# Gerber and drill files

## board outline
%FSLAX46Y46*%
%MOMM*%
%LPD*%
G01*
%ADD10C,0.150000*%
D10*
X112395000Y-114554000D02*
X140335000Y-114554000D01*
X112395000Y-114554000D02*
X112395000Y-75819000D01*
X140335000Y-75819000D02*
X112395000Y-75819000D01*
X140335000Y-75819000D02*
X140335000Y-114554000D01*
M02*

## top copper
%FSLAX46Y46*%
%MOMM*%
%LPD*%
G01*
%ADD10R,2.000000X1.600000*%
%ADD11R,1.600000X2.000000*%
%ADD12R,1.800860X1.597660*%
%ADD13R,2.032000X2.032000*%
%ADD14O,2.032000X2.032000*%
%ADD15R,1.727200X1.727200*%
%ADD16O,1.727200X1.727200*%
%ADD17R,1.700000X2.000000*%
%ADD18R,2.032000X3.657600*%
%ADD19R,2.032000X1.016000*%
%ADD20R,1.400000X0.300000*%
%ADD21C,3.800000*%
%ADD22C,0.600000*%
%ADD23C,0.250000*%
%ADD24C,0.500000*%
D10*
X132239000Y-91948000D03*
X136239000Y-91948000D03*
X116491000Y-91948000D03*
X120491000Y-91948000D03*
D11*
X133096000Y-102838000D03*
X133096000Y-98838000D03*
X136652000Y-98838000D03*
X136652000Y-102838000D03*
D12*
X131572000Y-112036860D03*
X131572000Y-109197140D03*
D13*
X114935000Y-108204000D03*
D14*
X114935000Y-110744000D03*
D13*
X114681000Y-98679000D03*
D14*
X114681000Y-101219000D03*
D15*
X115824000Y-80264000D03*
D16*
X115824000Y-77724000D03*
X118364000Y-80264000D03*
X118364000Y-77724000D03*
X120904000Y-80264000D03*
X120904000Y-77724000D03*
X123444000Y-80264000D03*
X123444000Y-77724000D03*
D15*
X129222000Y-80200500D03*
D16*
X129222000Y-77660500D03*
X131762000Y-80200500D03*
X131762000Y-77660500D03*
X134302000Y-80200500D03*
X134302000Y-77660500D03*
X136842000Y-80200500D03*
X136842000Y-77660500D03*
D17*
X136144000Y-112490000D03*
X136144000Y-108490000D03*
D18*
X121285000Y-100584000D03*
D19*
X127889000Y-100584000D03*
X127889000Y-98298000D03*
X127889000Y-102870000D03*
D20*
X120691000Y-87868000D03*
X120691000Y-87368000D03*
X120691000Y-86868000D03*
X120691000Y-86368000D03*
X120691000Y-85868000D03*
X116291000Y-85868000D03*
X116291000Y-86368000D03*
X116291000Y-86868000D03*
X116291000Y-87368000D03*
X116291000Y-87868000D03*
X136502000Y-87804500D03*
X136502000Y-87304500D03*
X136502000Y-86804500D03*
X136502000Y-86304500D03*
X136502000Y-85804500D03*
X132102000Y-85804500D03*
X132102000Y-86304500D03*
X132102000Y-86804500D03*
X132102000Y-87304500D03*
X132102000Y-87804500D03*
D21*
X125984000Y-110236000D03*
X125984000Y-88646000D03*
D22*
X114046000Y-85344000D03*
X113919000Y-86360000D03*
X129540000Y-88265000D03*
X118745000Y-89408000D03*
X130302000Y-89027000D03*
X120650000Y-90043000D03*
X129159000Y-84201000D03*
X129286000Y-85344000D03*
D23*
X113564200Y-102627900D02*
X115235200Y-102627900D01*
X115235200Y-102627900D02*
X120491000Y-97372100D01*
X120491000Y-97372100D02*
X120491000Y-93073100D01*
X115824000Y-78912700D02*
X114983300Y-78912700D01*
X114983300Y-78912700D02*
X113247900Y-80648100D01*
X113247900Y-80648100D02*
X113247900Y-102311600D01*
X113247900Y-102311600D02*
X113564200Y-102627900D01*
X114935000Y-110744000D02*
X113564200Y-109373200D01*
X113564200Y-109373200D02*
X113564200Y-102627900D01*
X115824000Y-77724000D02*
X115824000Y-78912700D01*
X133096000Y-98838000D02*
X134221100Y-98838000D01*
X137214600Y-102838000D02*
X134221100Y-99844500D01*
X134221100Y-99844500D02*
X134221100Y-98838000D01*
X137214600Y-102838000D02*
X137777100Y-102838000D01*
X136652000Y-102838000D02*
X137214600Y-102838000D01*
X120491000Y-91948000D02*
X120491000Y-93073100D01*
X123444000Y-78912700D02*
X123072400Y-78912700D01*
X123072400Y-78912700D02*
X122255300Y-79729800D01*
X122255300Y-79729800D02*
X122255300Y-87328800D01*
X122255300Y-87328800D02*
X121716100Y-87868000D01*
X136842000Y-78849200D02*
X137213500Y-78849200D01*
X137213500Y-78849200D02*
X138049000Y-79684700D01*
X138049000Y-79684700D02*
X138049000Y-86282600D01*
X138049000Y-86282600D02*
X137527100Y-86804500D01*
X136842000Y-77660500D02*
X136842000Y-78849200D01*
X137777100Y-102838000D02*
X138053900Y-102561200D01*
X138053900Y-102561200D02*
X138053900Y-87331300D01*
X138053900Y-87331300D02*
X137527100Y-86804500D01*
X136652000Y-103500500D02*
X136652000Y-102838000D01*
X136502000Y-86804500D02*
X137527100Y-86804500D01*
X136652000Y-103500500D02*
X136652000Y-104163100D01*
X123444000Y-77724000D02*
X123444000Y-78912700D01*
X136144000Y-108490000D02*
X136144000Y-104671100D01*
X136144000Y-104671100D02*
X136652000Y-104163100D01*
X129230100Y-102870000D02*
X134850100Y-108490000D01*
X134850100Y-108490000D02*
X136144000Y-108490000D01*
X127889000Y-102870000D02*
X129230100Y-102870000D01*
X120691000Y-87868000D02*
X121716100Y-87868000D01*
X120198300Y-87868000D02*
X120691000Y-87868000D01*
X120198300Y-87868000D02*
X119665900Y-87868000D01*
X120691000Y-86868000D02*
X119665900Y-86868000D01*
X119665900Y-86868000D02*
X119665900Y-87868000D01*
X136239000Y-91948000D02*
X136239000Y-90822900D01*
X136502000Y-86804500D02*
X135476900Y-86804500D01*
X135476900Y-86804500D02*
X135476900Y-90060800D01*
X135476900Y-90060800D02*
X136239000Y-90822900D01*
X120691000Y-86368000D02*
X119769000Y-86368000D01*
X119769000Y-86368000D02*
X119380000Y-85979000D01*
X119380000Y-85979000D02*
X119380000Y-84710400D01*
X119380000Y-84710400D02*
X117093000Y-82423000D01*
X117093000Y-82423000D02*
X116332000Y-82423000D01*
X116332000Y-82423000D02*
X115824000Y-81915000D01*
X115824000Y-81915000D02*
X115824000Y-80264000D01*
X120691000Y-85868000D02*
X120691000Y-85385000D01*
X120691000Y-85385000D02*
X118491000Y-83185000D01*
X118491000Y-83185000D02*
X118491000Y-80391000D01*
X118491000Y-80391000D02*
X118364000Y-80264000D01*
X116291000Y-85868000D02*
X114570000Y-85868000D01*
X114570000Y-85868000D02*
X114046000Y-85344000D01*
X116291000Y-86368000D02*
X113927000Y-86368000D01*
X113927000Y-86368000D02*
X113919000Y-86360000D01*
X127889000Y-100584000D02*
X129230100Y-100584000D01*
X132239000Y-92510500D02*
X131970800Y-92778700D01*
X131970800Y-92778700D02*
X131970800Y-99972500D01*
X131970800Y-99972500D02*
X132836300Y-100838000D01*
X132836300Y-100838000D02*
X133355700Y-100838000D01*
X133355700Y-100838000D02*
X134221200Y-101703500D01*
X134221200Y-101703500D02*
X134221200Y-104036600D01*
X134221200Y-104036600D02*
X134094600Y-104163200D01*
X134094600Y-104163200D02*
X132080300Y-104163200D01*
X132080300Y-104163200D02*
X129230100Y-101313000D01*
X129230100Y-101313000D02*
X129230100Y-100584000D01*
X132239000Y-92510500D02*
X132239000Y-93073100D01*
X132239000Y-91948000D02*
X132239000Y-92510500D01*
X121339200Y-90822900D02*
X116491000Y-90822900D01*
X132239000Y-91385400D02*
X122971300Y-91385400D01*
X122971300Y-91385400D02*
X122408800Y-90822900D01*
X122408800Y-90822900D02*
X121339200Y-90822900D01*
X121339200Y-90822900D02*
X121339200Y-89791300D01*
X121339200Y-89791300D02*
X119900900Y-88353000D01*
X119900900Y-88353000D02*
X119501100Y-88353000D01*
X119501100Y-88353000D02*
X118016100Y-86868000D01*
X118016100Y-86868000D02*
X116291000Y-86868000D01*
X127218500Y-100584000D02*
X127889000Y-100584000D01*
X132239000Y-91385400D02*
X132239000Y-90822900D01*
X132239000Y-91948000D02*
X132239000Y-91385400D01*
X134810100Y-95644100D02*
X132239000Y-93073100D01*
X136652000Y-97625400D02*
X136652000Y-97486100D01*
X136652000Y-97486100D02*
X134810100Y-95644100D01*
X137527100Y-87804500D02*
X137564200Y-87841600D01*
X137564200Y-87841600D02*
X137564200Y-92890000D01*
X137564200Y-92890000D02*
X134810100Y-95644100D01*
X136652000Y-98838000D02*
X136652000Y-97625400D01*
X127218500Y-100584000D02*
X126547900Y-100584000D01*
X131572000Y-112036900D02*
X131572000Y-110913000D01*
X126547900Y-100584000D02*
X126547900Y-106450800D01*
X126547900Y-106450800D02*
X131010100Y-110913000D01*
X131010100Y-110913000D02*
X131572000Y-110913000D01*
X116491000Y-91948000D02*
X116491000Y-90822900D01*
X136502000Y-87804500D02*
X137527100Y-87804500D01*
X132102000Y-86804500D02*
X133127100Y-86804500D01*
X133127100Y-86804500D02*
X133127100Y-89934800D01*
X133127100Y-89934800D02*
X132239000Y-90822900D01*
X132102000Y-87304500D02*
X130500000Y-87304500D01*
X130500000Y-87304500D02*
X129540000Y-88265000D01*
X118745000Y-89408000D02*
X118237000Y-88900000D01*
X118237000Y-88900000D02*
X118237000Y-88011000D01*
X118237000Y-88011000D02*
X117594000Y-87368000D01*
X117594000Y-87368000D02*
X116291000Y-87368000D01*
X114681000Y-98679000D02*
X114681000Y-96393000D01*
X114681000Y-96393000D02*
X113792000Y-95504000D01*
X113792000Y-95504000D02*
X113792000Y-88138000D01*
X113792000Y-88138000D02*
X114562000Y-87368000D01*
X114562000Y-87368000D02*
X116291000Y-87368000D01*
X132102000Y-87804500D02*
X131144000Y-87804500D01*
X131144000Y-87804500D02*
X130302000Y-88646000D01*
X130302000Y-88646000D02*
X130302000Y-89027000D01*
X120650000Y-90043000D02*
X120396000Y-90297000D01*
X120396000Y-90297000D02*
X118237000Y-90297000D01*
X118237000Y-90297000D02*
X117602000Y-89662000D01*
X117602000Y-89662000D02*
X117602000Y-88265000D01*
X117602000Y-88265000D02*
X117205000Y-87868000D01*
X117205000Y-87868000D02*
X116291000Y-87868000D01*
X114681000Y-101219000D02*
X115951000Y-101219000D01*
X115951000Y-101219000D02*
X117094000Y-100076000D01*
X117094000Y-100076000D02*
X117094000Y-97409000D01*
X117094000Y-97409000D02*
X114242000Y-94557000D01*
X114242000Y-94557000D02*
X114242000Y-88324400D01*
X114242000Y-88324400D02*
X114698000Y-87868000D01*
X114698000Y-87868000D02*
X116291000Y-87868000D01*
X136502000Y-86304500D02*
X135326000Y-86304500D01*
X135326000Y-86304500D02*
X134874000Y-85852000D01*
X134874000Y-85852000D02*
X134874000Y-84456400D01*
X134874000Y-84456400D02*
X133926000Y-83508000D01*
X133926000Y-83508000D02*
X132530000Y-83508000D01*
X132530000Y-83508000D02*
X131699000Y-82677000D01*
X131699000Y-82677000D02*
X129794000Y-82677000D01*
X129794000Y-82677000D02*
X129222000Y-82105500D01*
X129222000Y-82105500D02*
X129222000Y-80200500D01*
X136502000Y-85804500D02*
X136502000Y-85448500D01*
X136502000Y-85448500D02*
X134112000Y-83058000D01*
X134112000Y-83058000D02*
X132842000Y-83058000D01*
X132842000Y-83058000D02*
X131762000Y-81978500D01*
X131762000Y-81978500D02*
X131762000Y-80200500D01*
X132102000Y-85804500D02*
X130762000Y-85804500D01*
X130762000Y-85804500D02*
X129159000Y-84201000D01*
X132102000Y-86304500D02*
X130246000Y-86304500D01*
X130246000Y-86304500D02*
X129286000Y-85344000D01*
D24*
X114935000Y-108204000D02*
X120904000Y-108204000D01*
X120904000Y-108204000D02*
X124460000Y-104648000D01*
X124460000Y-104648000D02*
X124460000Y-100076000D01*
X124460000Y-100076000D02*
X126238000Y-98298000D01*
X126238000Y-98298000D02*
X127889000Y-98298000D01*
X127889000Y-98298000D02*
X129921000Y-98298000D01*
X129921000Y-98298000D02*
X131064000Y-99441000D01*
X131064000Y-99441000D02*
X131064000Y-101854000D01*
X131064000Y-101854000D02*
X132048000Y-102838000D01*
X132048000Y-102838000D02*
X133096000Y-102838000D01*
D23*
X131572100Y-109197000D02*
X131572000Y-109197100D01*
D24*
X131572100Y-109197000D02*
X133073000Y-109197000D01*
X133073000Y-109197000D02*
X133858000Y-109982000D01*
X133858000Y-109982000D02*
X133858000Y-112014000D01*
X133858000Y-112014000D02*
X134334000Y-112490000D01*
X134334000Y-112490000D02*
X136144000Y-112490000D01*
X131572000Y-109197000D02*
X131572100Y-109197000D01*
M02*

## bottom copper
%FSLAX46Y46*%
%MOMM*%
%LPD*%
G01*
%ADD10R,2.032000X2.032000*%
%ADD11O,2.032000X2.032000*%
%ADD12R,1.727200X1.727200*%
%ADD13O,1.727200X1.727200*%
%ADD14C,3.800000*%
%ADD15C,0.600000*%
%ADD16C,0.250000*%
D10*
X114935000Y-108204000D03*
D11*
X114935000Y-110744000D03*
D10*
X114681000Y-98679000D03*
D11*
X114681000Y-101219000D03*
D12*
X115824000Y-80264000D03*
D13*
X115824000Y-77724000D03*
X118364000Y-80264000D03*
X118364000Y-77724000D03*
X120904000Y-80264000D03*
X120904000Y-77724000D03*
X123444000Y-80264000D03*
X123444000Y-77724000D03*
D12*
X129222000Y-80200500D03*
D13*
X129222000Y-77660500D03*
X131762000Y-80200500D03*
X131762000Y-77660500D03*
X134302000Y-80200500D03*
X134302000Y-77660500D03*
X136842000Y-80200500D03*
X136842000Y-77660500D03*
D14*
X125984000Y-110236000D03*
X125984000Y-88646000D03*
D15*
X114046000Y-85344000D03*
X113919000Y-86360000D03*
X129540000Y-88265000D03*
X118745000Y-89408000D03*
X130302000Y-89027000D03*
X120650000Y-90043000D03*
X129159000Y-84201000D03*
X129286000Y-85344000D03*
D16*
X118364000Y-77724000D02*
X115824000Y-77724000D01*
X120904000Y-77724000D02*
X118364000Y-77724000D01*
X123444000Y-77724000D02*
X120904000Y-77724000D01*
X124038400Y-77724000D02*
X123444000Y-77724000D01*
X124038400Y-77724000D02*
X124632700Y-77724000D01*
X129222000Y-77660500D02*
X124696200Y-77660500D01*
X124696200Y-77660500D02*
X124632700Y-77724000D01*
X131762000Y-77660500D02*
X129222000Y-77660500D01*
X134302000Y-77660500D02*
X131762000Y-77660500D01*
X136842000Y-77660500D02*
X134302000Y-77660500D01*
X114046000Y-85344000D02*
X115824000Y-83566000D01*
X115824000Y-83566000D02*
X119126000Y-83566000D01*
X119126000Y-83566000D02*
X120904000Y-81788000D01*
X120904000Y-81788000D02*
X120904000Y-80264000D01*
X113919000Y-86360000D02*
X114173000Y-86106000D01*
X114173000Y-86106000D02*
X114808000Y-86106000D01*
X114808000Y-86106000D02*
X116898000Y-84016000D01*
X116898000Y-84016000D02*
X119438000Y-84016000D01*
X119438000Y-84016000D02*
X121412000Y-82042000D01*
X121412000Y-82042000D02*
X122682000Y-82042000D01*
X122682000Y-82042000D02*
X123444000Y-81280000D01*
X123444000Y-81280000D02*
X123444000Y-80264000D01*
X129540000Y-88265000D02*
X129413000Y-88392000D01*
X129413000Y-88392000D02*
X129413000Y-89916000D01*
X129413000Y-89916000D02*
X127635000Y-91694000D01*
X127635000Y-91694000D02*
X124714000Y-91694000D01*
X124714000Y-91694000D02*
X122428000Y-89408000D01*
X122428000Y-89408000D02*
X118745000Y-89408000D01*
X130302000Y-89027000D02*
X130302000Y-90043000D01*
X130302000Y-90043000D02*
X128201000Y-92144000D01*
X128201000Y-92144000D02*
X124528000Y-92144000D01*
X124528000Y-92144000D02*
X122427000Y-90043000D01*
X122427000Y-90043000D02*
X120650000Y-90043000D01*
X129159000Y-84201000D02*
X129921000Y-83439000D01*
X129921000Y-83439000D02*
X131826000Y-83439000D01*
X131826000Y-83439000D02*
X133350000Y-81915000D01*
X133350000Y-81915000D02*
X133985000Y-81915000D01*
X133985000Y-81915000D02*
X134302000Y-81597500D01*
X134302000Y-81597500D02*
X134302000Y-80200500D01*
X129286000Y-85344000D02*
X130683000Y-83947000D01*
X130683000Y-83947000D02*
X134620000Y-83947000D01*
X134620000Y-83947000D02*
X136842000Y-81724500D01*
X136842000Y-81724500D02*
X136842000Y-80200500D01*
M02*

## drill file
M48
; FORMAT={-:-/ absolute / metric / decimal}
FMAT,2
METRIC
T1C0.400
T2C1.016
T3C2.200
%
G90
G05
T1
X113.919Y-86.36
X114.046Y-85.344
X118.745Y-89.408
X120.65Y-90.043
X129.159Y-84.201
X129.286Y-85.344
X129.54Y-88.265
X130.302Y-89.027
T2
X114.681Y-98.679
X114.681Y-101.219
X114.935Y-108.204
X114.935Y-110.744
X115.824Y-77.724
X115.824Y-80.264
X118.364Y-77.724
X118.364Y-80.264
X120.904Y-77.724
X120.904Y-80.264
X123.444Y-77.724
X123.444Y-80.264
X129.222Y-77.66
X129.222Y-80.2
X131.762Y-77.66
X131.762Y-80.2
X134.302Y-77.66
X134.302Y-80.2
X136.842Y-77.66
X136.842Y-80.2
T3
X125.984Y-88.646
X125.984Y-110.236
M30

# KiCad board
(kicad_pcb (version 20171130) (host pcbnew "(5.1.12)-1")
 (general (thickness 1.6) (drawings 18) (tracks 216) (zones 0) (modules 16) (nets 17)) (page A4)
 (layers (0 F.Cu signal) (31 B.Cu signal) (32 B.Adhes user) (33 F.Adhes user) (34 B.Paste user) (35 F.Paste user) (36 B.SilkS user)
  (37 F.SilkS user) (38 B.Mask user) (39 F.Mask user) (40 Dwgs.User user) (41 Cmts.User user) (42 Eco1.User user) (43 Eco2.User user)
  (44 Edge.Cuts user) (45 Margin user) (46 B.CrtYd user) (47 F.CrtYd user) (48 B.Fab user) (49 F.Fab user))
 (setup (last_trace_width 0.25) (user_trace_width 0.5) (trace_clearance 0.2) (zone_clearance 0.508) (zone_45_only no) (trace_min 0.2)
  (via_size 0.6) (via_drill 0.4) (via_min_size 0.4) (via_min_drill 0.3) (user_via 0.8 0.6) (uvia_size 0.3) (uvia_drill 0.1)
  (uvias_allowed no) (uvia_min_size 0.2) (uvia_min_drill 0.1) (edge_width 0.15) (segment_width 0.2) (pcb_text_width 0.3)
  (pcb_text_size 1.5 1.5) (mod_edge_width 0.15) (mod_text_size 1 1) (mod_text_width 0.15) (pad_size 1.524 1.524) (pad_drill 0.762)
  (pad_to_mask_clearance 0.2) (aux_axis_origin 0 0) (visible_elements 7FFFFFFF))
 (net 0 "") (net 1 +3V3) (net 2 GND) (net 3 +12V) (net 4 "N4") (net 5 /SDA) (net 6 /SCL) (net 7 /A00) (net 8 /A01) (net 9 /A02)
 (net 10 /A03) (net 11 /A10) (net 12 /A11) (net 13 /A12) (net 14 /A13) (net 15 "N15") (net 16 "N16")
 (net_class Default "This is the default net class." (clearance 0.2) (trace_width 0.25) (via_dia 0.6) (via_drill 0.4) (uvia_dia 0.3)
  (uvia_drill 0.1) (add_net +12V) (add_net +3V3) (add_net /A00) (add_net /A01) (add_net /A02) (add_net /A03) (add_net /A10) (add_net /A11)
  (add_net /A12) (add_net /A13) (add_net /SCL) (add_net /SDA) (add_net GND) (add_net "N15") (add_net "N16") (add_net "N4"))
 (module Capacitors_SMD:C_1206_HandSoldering (layer F.Cu) (at 134.239 91.948)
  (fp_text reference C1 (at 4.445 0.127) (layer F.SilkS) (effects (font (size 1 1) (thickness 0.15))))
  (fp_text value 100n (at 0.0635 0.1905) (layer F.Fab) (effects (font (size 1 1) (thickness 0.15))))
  (pad 1 smd rect (at -2 0) (size 2 1.6) (layers F.Cu F.Paste F.Mask) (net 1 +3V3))
  (pad 2 smd rect (at 2 0) (size 2 1.6) (layers F.Cu F.Paste F.Mask) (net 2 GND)))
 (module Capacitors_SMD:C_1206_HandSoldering (layer F.Cu) (at 118.491 91.948)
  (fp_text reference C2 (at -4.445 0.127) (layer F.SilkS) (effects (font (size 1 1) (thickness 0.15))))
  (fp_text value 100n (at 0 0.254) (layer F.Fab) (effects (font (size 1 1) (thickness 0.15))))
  (pad 1 smd rect (at -2 0) (size 2 1.6) (layers F.Cu F.Paste F.Mask) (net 1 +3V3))
  (pad 2 smd rect (at 2 0) (size 2 1.6) (layers F.Cu F.Paste F.Mask) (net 2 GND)))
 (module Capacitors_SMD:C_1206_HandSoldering (layer F.Cu) (at 133.096 100.838 90)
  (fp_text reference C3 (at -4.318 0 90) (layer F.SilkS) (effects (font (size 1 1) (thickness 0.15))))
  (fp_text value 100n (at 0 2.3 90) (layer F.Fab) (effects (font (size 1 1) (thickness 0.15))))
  (pad 1 smd rect (at -2 0 90) (size 2 1.6) (layers F.Cu F.Paste F.Mask) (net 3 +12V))
  (pad 2 smd rect (at 2 0 90) (size 2 1.6) (layers F.Cu F.Paste F.Mask) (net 2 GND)))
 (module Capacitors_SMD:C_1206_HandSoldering (layer F.Cu) (at 136.652 100.838 270)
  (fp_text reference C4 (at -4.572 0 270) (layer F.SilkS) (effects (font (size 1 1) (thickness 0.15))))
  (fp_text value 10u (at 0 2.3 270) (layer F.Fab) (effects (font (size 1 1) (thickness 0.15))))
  (pad 1 smd rect (at -2 0 270) (size 2 1.6) (layers F.Cu F.Paste F.Mask) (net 1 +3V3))
  (pad 2 smd rect (at 2 0 270) (size 2 1.6) (layers F.Cu F.Paste F.Mask) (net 2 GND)))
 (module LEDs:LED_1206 (layer F.Cu) (at 131.572 110.617 270)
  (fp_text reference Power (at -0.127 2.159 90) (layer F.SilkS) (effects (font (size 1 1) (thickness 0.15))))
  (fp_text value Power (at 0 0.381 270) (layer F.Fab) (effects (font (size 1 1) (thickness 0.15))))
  (pad 2 smd rect (at 1.41986 0 90) (size 1.59766 1.80086) (layers F.Cu F.Paste F.Mask) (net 1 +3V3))
  (pad 1 smd rect (at -1.41986 0 90) (size 1.59766 1.80086) (layers F.Cu F.Paste F.Mask) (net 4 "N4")))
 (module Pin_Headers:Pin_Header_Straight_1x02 (layer F.Cu) (at 114.935 108.204)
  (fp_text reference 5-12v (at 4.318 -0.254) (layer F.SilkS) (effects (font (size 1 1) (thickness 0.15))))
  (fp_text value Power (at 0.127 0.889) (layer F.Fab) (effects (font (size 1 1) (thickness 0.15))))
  (pad 1 thru_hole rect (at 0 0) (size 2.032 2.032) (drill 1.016) (layers *.Cu *.Mask F.SilkS) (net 3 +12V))
  (pad 2 thru_hole oval (at 0 2.54) (size 2.032 2.032) (drill 1.016) (layers *.Cu *.Mask F.SilkS) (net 2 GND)))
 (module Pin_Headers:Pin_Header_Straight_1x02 (layer F.Cu) (at 114.681 98.679)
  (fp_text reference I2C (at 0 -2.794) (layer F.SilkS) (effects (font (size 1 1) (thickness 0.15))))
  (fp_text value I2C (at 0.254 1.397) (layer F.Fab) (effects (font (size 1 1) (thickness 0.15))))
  (pad 1 thru_hole rect (at 0 0) (size 2.032 2.032) (drill 1.016) (layers *.Cu *.Mask F.SilkS) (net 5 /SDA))
  (pad 2 thru_hole oval (at 0 2.54) (size 2.032 2.032) (drill 1.016) (layers *.Cu *.Mask F.SilkS) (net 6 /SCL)))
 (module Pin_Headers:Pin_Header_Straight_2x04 (layer F.Cu) (at 115.824 80.264 90)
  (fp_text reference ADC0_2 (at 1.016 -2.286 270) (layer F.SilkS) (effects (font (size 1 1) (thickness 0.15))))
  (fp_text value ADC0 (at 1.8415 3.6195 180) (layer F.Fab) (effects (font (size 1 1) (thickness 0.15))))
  (pad 1 thru_hole rect (at 0 0 90) (size 1.7272 1.7272) (drill 1.016) (layers *.Cu *.Mask F.SilkS) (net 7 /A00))
  (pad 2 thru_hole oval (at 2.54 0 90) (size 1.7272 1.7272) (drill 1.016) (layers *.Cu *.Mask F.SilkS) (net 2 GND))
  (pad 3 thru_hole oval (at 0 2.54 90) (size 1.7272 1.7272) (drill 1.016) (layers *.Cu *.Mask F.SilkS) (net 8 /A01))
  (pad 4 thru_hole oval (at 2.54 2.54 90) (size 1.7272 1.7272) (drill 1.016) (layers *.Cu *.Mask F.SilkS) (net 2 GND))
  (pad 5 thru_hole oval (at 0 5.08 90) (size 1.7272 1.7272) (drill 1.016) (layers *.Cu *.Mask F.SilkS) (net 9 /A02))
  (pad 6 thru_hole oval (at 2.54 5.08 90) (size 1.7272 1.7272) (drill 1.016) (layers *.Cu *.Mask F.SilkS) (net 2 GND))
  (pad 7 thru_hole oval (at 0 7.62 90) (size 1.7272 1.7272) (drill 1.016) (layers *.Cu *.Mask F.SilkS) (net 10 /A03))
  (pad 8 thru_hole oval (at 2.54 7.62 90) (size 1.7272 1.7272) (drill 1.016) (layers *.Cu *.Mask F.SilkS) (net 2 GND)))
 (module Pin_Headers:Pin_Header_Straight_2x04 (layer F.Cu) (at 129.222 80.2005 90)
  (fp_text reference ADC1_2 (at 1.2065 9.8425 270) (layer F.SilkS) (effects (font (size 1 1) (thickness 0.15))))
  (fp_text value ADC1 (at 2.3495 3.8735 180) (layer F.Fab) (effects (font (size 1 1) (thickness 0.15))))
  (pad 1 thru_hole rect (at 0 0 90) (size 1.7272 1.7272) (drill 1.016) (layers *.Cu *.Mask F.SilkS) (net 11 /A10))
  (pad 2 thru_hole oval (at 2.54 0 90) (size 1.7272 1.7272) (drill 1.016) (layers *.Cu *.Mask F.SilkS) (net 2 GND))
  (pad 3 thru_hole oval (at 0 2.54 90) (size 1.7272 1.7272) (drill 1.016) (layers *.Cu *.Mask F.SilkS) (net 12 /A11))
  (pad 4 thru_hole oval (at 2.54 2.54 90) (size 1.7272 1.7272) (drill 1.016) (layers *.Cu *.Mask F.SilkS) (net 2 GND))
  (pad 5 thru_hole oval (at 0 5.08 90) (size 1.7272 1.7272) (drill 1.016) (layers *.Cu *.Mask F.SilkS) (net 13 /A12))
  (pad 6 thru_hole oval (at 2.54 5.08 90) (size 1.7272 1.7272) (drill 1.016) (layers *.Cu *.Mask F.SilkS) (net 2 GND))
  (pad 7 thru_hole oval (at 0 7.62 90) (size 1.7272 1.7272) (drill 1.016) (layers *.Cu *.Mask F.SilkS) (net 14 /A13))
  (pad 8 thru_hole oval (at 2.54 7.62 90) (size 1.7272 1.7272) (drill 1.016) (layers *.Cu *.Mask F.SilkS) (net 2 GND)))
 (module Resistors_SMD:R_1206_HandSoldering (layer F.Cu) (at 136.144 110.49 90)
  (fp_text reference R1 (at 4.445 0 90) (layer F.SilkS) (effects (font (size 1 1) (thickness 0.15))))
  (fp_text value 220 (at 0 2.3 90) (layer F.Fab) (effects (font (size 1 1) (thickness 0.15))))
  (pad 1 smd rect (at -2 0 90) (size 2 1.7) (layers F.Cu F.Paste F.Mask) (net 4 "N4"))
  (pad 2 smd rect (at 2 0 90) (size 2 1.7) (layers F.Cu F.Paste F.Mask) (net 2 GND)))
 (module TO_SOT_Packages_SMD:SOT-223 (layer F.Cu) (at 124.587 100.584 90)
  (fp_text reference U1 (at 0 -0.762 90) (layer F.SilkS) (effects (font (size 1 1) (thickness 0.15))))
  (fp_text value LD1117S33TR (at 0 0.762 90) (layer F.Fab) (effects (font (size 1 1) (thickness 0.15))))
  (pad 4 smd rect (at 0 -3.302 90) (size 3.6576 2.032) (layers F.Cu F.Paste F.Mask))
  (pad 2 smd rect (at 0 3.302 90) (size 1.016 2.032) (layers F.Cu F.Paste F.Mask) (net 1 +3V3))
  (pad 3 smd rect (at 2.286 3.302 90) (size 1.016 2.032) (layers F.Cu F.Paste F.Mask) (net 3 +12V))
  (pad 1 smd rect (at -2.286 3.302 90) (size 1.016 2.032) (layers F.Cu F.Paste F.Mask) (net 2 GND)))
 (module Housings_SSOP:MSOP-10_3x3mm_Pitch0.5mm (layer F.Cu) (at 118.491 86.868 180)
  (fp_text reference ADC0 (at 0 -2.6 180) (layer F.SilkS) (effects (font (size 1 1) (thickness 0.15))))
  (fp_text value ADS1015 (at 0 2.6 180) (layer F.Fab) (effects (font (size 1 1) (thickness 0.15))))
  (pad 1 smd rect (at -2.2 -1 180) (size 1.4 0.3) (layers F.Cu F.Paste F.Mask) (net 2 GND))
  (pad 2 smd rect (at -2.2 -0.5 180) (size 1.4 0.3) (layers F.Cu F.Paste F.Mask) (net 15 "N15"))
  (pad 3 smd rect (at -2.2 0 180) (size 1.4 0.3) (layers F.Cu F.Paste F.Mask) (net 2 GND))
  (pad 4 smd rect (at -2.2 0.5 180) (size 1.4 0.3) (layers F.Cu F.Paste F.Mask) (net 7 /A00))
  (pad 5 smd rect (at -2.2 1 180) (size 1.4 0.3) (layers F.Cu F.Paste F.Mask) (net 8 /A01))
  (pad 6 smd rect (at 2.2 1 180) (size 1.4 0.3) (layers F.Cu F.Paste F.Mask) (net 9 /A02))
  (pad 7 smd rect (at 2.2 0.5 180) (size 1.4 0.3) (layers F.Cu F.Paste F.Mask) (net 10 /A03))
  (pad 8 smd rect (at 2.2 0 180) (size 1.4 0.3) (layers F.Cu F.Paste F.Mask) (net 1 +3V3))
  (pad 9 smd rect (at 2.2 -0.5 180) (size 1.4 0.3) (layers F.Cu F.Paste F.Mask) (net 5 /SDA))
  (pad 10 smd rect (at 2.2 -1 180) (size 1.4 0.3) (layers F.Cu F.Paste F.Mask) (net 6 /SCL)))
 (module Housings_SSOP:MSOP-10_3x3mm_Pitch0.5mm (layer F.Cu) (at 134.302 86.8045 180)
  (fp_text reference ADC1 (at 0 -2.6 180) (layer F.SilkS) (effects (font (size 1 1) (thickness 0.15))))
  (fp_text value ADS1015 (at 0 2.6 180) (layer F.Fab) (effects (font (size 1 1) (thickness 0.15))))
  (pad 1 smd rect (at -2.2 -1 180) (size 1.4 0.3) (layers F.Cu F.Paste F.Mask) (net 1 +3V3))
  (pad 2 smd rect (at -2.2 -0.5 180) (size 1.4 0.3) (layers F.Cu F.Paste F.Mask) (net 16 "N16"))
  (pad 3 smd rect (at -2.2 0 180) (size 1.4 0.3) (layers F.Cu F.Paste F.Mask) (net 2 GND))
  (pad 4 smd rect (at -2.2 0.5 180) (size 1.4 0.3) (layers F.Cu F.Paste F.Mask) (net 11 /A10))
  (pad 5 smd rect (at -2.2 1 180) (size 1.4 0.3) (layers F.Cu F.Paste F.Mask) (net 12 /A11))
  (pad 6 smd rect (at 2.2 1 180) (size 1.4 0.3) (layers F.Cu F.Paste F.Mask) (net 13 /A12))
  (pad 7 smd rect (at 2.2 0.5 180) (size 1.4 0.3) (layers F.Cu F.Paste F.Mask) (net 14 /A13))
  (pad 8 smd rect (at 2.2 0 180) (size 1.4 0.3) (layers F.Cu F.Paste F.Mask) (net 1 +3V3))
  (pad 9 smd rect (at 2.2 -0.5 180) (size 1.4 0.3) (layers F.Cu F.Paste F.Mask) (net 5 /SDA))
  (pad 10 smd rect (at 2.2 -1 180) (size 1.4 0.3) (layers F.Cu F.Paste F.Mask) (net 6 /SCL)))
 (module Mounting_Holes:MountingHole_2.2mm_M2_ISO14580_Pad (layer F.Cu) (at 125.984 110.236)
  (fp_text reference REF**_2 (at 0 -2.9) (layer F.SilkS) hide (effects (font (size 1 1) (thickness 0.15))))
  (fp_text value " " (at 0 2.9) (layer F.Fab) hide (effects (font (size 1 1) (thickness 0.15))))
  (pad 1 thru_hole circle (at 0 0) (size 3.8 3.8) (drill 2.2) (layers *.Cu *.Mask F.SilkS)))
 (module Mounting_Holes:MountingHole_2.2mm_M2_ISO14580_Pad (layer F.Cu) (at 125.984 88.646)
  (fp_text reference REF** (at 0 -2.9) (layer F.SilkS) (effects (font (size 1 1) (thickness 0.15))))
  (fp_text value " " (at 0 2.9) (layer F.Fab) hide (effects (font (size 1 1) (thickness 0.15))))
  (pad 1 thru_hole circle (at 0 0) (size 3.8 3.8) (drill 2.2) (layers *.Cu *.Mask F.SilkS)))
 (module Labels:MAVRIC (layer B.Cu) (at 127.889 100.076 90)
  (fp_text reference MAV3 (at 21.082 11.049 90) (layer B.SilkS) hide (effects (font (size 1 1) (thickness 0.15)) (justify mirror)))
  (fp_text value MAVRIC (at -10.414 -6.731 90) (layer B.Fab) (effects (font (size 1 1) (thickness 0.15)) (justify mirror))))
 (gr_line (start 112.395 114.554) (end 140.335 114.554) (angle 90) (layer Edge.Cuts) (width 0.15))
 (gr_line (start 112.395 114.554) (end 112.395 75.819) (angle 90) (layer Edge.Cuts) (width 0.15))
 (gr_line (start 140.335 75.819) (end 112.395 75.819) (angle 90) (layer Edge.Cuts) (width 0.15))
 (gr_line (start 140.335 75.819) (end 140.335 114.554) (angle 90) (layer Edge.Cuts) (width 0.15))
 (segment (start 113.5642 102.6279) (end 115.2352 102.6279) (width 0.25) (layer F.Cu) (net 2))
 (segment (start 115.2352 102.6279) (end 120.491 97.3721) (width 0.25) (layer F.Cu) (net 2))
 (segment (start 120.491 97.3721) (end 120.491 93.0731) (width 0.25) (layer F.Cu) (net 2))
 (segment (start 115.824 78.9127) (end 114.9833 78.9127) (width 0.25) (layer F.Cu) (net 2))
 (segment (start 114.9833 78.9127) (end 113.2479 80.6481) (width 0.25) (layer F.Cu) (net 2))
 (segment (start 113.2479 80.6481) (end 113.2479 102.3116) (width 0.25) (layer F.Cu) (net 2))
 (segment (start 113.2479 102.3116) (end 113.5642 102.6279) (width 0.25) (layer F.Cu) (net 2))
 (segment (start 114.935 110.744) (end 113.5642 109.3732) (width 0.25) (layer F.Cu) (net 2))
 (segment (start 113.5642 109.3732) (end 113.5642 102.6279) (width 0.25) (layer F.Cu) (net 2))
 (segment (start 115.824 77.724) (end 115.824 78.9127) (width 0.25) (layer F.Cu) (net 2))
 (segment (start 133.096 98.838) (end 134.2211 98.838) (width 0.25) (layer F.Cu) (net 2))
 (segment (start 137.2146 102.838) (end 134.2211 99.8445) (width 0.25) (layer F.Cu) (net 2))
 (segment (start 134.2211 99.8445) (end 134.2211 98.838) (width 0.25) (layer F.Cu) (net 2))
 (segment (start 137.2146 102.838) (end 137.7771 102.838) (width 0.25) (layer F.Cu) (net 2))
 (segment (start 136.652 102.838) (end 137.2146 102.838) (width 0.25) (layer F.Cu) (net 2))
 (segment (start 120.491 91.948) (end 120.491 93.0731) (width 0.25) (layer F.Cu) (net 2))
 (segment (start 123.444 78.9127) (end 123.0724 78.9127) (width 0.25) (layer F.Cu) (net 2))
 (segment (start 123.0724 78.9127) (end 122.2553 79.7298) (width 0.25) (layer F.Cu) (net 2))
 (segment (start 122.2553 79.7298) (end 122.2553 87.3288) (width 0.25) (layer F.Cu) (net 2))
 (segment (start 122.2553 87.3288) (end 121.7161 87.868) (width 0.25) (layer F.Cu) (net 2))
 (segment (start 136.842 78.8492) (end 137.2135 78.8492) (width 0.25) (layer F.Cu) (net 2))
 (segment (start 137.2135 78.8492) (end 138.049 79.6847) (width 0.25) (layer F.Cu) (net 2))
 (segment (start 138.049 79.6847) (end 138.049 86.2826) (width 0.25) (layer F.Cu) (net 2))
 (segment (start 138.049 86.2826) (end 137.5271 86.8045) (width 0.25) (layer F.Cu) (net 2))
 (segment (start 136.842 77.6605) (end 136.842 78.8492) (width 0.25) (layer F.Cu) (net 2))
 (segment (start 137.7771 102.838) (end 138.0539 102.5612) (width 0.25) (layer F.Cu) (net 2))
 (segment (start 138.0539 102.5612) (end 138.0539 87.3313) (width 0.25) (layer F.Cu) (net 2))
 (segment (start 138.0539 87.3313) (end 137.5271 86.8045) (width 0.25) (layer F.Cu) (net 2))
 (segment (start 136.652 103.5005) (end 136.652 102.838) (width 0.25) (layer F.Cu) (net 2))
 (segment (start 136.502 86.8045) (end 137.5271 86.8045) (width 0.25) (layer F.Cu) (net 2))
 (segment (start 136.652 103.5005) (end 136.652 104.1631) (width 0.25) (layer F.Cu) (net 2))
 (segment (start 123.444 77.724) (end 123.444 78.9127) (width 0.25) (layer F.Cu) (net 2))
 (segment (start 118.364 77.724) (end 115.824 77.724) (width 0.25) (layer B.Cu) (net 2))
 (segment (start 120.904 77.724) (end 118.364 77.724) (width 0.25) (layer B.Cu) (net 2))
 (segment (start 123.444 77.724) (end 120.904 77.724) (width 0.25) (layer B.Cu) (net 2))
 (segment (start 124.0384 77.724) (end 123.444 77.724) (width 0.25) (layer B.Cu) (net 2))
 (segment (start 124.0384 77.724) (end 124.6327 77.724) (width 0.25) (layer B.Cu) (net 2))
 (segment (start 129.222 77.6605) (end 124.6962 77.6605) (width 0.25) (layer B.Cu) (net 2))
 (segment (start 124.6962 77.6605) (end 124.6327 77.724) (width 0.25) (layer B.Cu) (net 2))
 (segment (start 131.762 77.6605) (end 129.222 77.6605) (width 0.25) (layer B.Cu) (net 2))
 (segment (start 134.302 77.6605) (end 131.762 77.6605) (width 0.25) (layer B.Cu) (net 2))
 (segment (start 136.842 77.6605) (end 134.302 77.6605) (width 0.25) (layer B.Cu) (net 2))
 (segment (start 136.144 108.49) (end 136.144 104.6711) (width 0.25) (layer F.Cu) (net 2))
 (segment (start 136.144 104.6711) (end 136.652 104.1631) (width 0.25) (layer F.Cu) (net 2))
 (segment (start 129.2301 102.87) (end 134.8501 108.49) (width 0.25) (layer F.Cu) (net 2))
 (segment (start 134.8501 108.49) (end 136.144 108.49) (width 0.25) (layer F.Cu) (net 2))
 (segment (start 127.889 102.87) (end 129.2301 102.87) (width 0.25) (layer F.Cu) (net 2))
 (segment (start 120.691 87.868) (end 121.7161 87.868) (width 0.25) (layer F.Cu) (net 2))
 (segment (start 120.1983 87.868) (end 120.691 87.868) (width 0.25) (layer F.Cu) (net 2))
 (segment (start 120.1983 87.868) (end 119.6659 87.868) (width 0.25) (layer F.Cu) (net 2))
 (segment (start 120.691 86.868) (end 119.6659 86.868) (width 0.25) (layer F.Cu) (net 2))
 (segment (start 119.6659 86.868) (end 119.6659 87.868) (width 0.25) (layer F.Cu) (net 2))
 (segment (start 136.239 91.948) (end 136.239 90.8229) (width 0.25) (layer F.Cu) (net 2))
 (segment (start 136.502 86.8045) (end 135.4769 86.8045) (width 0.25) (layer F.Cu) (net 2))
 (segment (start 135.4769 86.8045) (end 135.4769 90.0608) (width 0.25) (layer F.Cu) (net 2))
 (segment (start 135.4769 90.0608) (end 136.239 90.8229) (width 0.25) (layer F.Cu) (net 2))
 (segment (start 120.691 86.368) (end 119.769 86.368) (width 0.25) (layer F.Cu) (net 7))
 (segment (start 119.769 86.368) (end 119.38 85.979) (width 0.25) (layer F.Cu) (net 7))
 (segment (start 119.38 85.979) (end 119.38 84.7104) (width 0.25) (layer F.Cu) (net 7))
 (segment (start 119.38 84.7104) (end 117.093 82.423) (width 0.25) (layer F.Cu) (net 7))
 (segment (start 117.093 82.423) (end 116.332 82.423) (width 0.25) (layer F.Cu) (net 7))
 (segment (start 116.332 82.423) (end 115.824 81.915) (width 0.25) (layer F.Cu) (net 7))
 (segment (start 115.824 81.915) (end 115.824 80.264) (width 0.25) (layer F.Cu) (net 7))
 (segment (start 120.691 85.868) (end 120.691 85.385) (width 0.25) (layer F.Cu) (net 8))
 (segment (start 120.691 85.385) (end 118.491 83.185) (width 0.25) (layer F.Cu) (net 8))
 (segment (start 118.491 83.185) (end 118.491 80.391) (width 0.25) (layer F.Cu) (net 8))
 (segment (start 118.491 80.391) (end 118.364 80.264) (width 0.25) (layer F.Cu) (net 8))
 (segment (start 116.291 85.868) (end 114.57 85.868) (width 0.25) (layer F.Cu) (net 9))
 (segment (start 114.57 85.868) (end 114.046 85.344) (width 0.25) (layer F.Cu) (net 9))
 (segment (start 114.046 85.344) (end 115.824 83.566) (width 0.25) (layer B.Cu) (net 9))
 (segment (start 115.824 83.566) (end 119.126 83.566) (width 0.25) (layer B.Cu) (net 9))
 (segment (start 119.126 83.566) (end 120.904 81.788) (width 0.25) (layer B.Cu) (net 9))
 (segment (start 120.904 81.788) (end 120.904 80.264) (width 0.25) (layer B.Cu) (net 9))
 (via (at 114.046 85.344) (size 0.6) (layers F.Cu B.Cu) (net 9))
 (segment (start 116.291 86.368) (end 113.927 86.368) (width 0.25) (layer F.Cu) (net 10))
 (segment (start 113.927 86.368) (end 113.919 86.36) (width 0.25) (layer F.Cu) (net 10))
 (segment (start 113.919 86.36) (end 114.173 86.106) (width 0.25) (layer B.Cu) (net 10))
 (segment (start 114.173 86.106) (end 114.808 86.106) (width 0.25) (layer B.Cu) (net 10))
 (segment (start 114.808 86.106) (end 116.898 84.016) (width 0.25) (layer B.Cu) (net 10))
 (segment (start 116.898 84.016) (end 119.438 84.016) (width 0.25) (layer B.Cu) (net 10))
 (segment (start 119.438 84.016) (end 121.412 82.042) (width 0.25) (layer B.Cu) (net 10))
 (segment (start 121.412 82.042) (end 122.682 82.042) (width 0.25) (layer B.Cu) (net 10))
 (segment (start 122.682 82.042) (end 123.444 81.28) (width 0.25) (layer B.Cu) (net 10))
 (segment (start 123.444 81.28) (end 123.444 80.264) (width 0.25) (layer B.Cu) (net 10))
 (via (at 113.919 86.36) (size 0.6) (layers F.Cu B.Cu) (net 10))
 (segment (start 127.889 100.584) (end 129.2301 100.584) (width 0.25) (layer F.Cu) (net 1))
 (segment (start 132.239 92.5105) (end 131.9708 92.7787) (width 0.25) (layer F.Cu) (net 1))
 (segment (start 131.9708 92.7787) (end 131.9708 99.9725) (width 0.25) (layer F.Cu) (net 1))
 (segment (start 131.9708 99.9725) (end 132.8363 100.838) (width 0.25) (layer F.Cu) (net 1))
 (segment (start 132.8363 100.838) (end 133.3557 100.838) (width 0.25) (layer F.Cu) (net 1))
 (segment (start 133.3557 100.838) (end 134.2212 101.7035) (width 0.25) (layer F.Cu) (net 1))
 (segment (start 134.2212 101.7035) (end 134.2212 104.0366) (width 0.25) (layer F.Cu) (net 1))
 (segment (start 134.2212 104.0366) (end 134.0946 104.1632) (width 0.25) (layer F.Cu) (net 1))
 (segment (start 134.0946 104.1632) (end 132.0803 104.1632) (width 0.25) (layer F.Cu) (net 1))
 (segment (start 132.0803 104.1632) (end 129.2301 101.313) (width 0.25) (layer F.Cu) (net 1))
 (segment (start 129.2301 101.313) (end 129.2301 100.584) (width 0.25) (layer F.Cu) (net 1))
 (segment (start 132.239 92.5105) (end 132.239 93.0731) (width 0.25) (layer F.Cu) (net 1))
 (segment (start 132.239 91.948) (end 132.239 92.5105) (width 0.25) (layer F.Cu) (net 1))
 (segment (start 121.3392 90.8229) (end 116.491 90.8229) (width 0.25) (layer F.Cu) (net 1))
 (segment (start 132.239 91.3854) (end 122.9713 91.3854) (width 0.25) (layer F.Cu) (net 1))
 (segment (start 122.9713 91.3854) (end 122.4088 90.8229) (width 0.25) (layer F.Cu) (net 1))
 (segment (start 122.4088 90.8229) (end 121.3392 90.8229) (width 0.25) (layer F.Cu) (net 1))
 (segment (start 121.3392 90.8229) (end 121.3392 89.7913) (width 0.25) (layer F.Cu) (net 1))
 (segment (start 121.3392 89.7913) (end 119.9009 88.353) (width 0.25) (layer F.Cu) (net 1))
 (segment (start 119.9009 88.353) (end 119.5011 88.353) (width 0.25) (layer F.Cu) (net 1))
 (segment (start 119.5011 88.353) (end 118.0161 86.868) (width 0.25) (layer F.Cu) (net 1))
 (segment (start 118.0161 86.868) (end 116.291 86.868) (width 0.25) (layer F.Cu) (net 1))
 (segment (start 127.2185 100.584) (end 127.889 100.584) (width 0.25) (layer F.Cu) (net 1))
 (segment (start 132.239 91.3854) (end 132.239 90.8229) (width 0.25) (layer F.Cu) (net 1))
 (segment (start 132.239 91.948) (end 132.239 91.3854) (width 0.25) (layer F.Cu) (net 1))
 (segment (start 134.8101 95.6441) (end 132.239 93.0731) (width 0.25) (layer F.Cu) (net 1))
 (segment (start 136.652 97.6254) (end 136.652 97.4861) (width 0.25) (layer F.Cu) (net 1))
 (segment (start 136.652 97.4861) (end 134.8101 95.6441) (width 0.25) (layer F.Cu) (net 1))
 (segment (start 137.5271 87.8045) (end 137.5642 87.8416) (width 0.25) (layer F.Cu) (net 1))
 (segment (start 137.5642 87.8416) (end 137.5642 92.89) (width 0.25) (layer F.Cu) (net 1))
 (segment (start 137.5642 92.89) (end 134.8101 95.6441) (width 0.25) (layer F.Cu) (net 1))
 (segment (start 136.652 98.838) (end 136.652 97.6254) (width 0.25) (layer F.Cu) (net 1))
 (segment (start 127.2185 100.584) (end 126.5479 100.584) (width 0.25) (layer F.Cu) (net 1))
 (segment (start 131.572 112.0369) (end 131.572 110.913) (width 0.25) (layer F.Cu) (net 1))
 (segment (start 126.5479 100.584) (end 126.5479 106.4508) (width 0.25) (layer F.Cu) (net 1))
 (segment (start 126.5479 106.4508) (end 131.0101 110.913) (width 0.25) (layer F.Cu) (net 1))
 (segment (start 131.0101 110.913) (end 131.572 110.913) (width 0.25) (layer F.Cu) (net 1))
 (segment (start 116.491 91.948) (end 116.491 90.8229) (width 0.25) (layer F.Cu) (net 1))
 (segment (start 136.502 87.8045) (end 137.5271 87.8045) (width 0.25) (layer F.Cu) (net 1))
 (segment (start 132.102 86.8045) (end 133.1271 86.8045) (width 0.25) (layer F.Cu) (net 1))
 (segment (start 133.1271 86.8045) (end 133.1271 89.9348) (width 0.25) (layer F.Cu) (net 1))
 (segment (start 133.1271 89.9348) (end 132.239 90.8229) (width 0.25) (layer F.Cu) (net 1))
 (segment (start 132.102 87.3045) (end 130.5 87.3045) (width 0.25) (layer F.Cu) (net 5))
 (segment (start 130.5 87.3045) (end 129.54 88.265) (width 0.25) (layer F.Cu) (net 5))
 (segment (start 129.54 88.265) (end 129.413 88.392) (width 0.25) (layer B.Cu) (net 5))
 (segment (start 129.413 88.392) (end 129.413 89.916) (width 0.25) (layer B.Cu) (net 5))
 (segment (start 129.413 89.916) (end 127.635 91.694) (width 0.25) (layer B.Cu) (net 5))
 (segment (start 127.635 91.694) (end 124.714 91.694) (width 0.25) (layer B.Cu) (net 5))
 (segment (start 124.714 91.694) (end 122.428 89.408) (width 0.25) (layer B.Cu) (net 5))
 (segment (start 122.428 89.408) (end 118.745 89.408) (width 0.25) (layer B.Cu) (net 5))
 (segment (start 118.745 89.408) (end 118.237 88.9) (width 0.25) (layer F.Cu) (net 5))
 (segment (start 118.237 88.9) (end 118.237 88.011) (width 0.25) (layer F.Cu) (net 5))
 (segment (start 118.237 88.011) (end 117.594 87.368) (width 0.25) (layer F.Cu) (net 5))
 (segment (start 117.594 87.368) (end 116.291 87.368) (width 0.25) (layer F.Cu) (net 5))
 (segment (start 114.681 98.679) (end 114.681 96.393) (width 0.25) (layer F.Cu) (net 5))
 (segment (start 114.681 96.393) (end 113.792 95.504) (width 0.25) (layer F.Cu) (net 5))
 (segment (start 113.792 95.504) (end 113.792 88.138) (width 0.25) (layer F.Cu) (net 5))
 (segment (start 113.792 88.138) (end 114.562 87.368) (width 0.25) (layer F.Cu) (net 5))
 (segment (start 114.562 87.368) (end 116.291 87.368) (width 0.25) (layer F.Cu) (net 5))
 (via (at 129.54 88.265) (size 0.6) (layers F.Cu B.Cu) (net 5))
 (via (at 118.745 89.408) (size 0.6) (layers F.Cu B.Cu) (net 5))
 (segment (start 132.102 87.8045) (end 131.144 87.8045) (width 0.25) (layer F.Cu) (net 6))
 (segment (start 131.144 87.8045) (end 130.302 88.646) (width 0.25) (layer F.Cu) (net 6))
 (segment (start 130.302 88.646) (end 130.302 89.027) (width 0.25) (layer F.Cu) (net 6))
 (segment (start 130.302 89.027) (end 130.302 90.043) (width 0.25) (layer B.Cu) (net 6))
 (segment (start 130.302 90.043) (end 128.201 92.144) (width 0.25) (layer B.Cu) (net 6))
 (segment (start 128.201 92.144) (end 124.528 92.144) (width 0.25) (layer B.Cu) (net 6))
 (segment (start 124.528 92.144) (end 122.427 90.043) (width 0.25) (layer B.Cu) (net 6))
 (segment (start 122.427 90.043) (end 120.65 90.043) (width 0.25) (layer B.Cu) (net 6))
 (segment (start 120.65 90.043) (end 120.396 90.297) (width 0.25) (layer F.Cu) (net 6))
 (segment (start 120.396 90.297) (end 118.237 90.297) (width 0.25) (layer F.Cu) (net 6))
 (segment (start 118.237 90.297) (end 117.602 89.662) (width 0.25) (layer F.Cu) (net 6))
 (segment (start 117.602 89.662) (end 117.602 88.265) (width 0.25) (layer F.Cu) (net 6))
 (segment (start 117.602 88.265) (end 117.205 87.868) (width 0.25) (layer F.Cu) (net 6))
 (segment (start 117.205 87.868) (end 116.291 87.868) (width 0.25) (layer F.Cu) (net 6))
 (segment (start 114.681 101.219) (end 115.951 101.219) (width 0.25) (layer F.Cu) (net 6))
 (segment (start 115.951 101.219) (end 117.094 100.076) (width 0.25) (layer F.Cu) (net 6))
 (segment (start 117.094 100.076) (end 117.094 97.409) (width 0.25) (layer F.Cu) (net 6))
 (segment (start 117.094 97.409) (end 114.242 94.557) (width 0.25) (layer F.Cu) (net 6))
 (segment (start 114.242 94.557) (end 114.242 88.3244) (width 0.25) (layer F.Cu) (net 6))
 (segment (start 114.242 88.3244) (end 114.698 87.868) (width 0.25) (layer F.Cu) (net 6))
 (segment (start 114.698 87.868) (end 116.291 87.868) (width 0.25) (layer F.Cu) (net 6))
 (via (at 130.302 89.027) (size 0.6) (layers F.Cu B.Cu) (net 6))
 (via (at 120.65 90.043) (size 0.6) (layers F.Cu B.Cu) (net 6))
 (segment (start 136.502 86.3045) (end 135.326 86.3045) (width 0.25) (layer F.Cu) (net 11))
 (segment (start 135.326 86.3045) (end 134.874 85.852) (width 0.25) (layer F.Cu) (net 11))
 (segment (start 134.874 85.852) (end 134.874 84.4564) (width 0.25) (layer F.Cu) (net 11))
 (segment (start 134.874 84.4564) (end 133.926 83.508) (width 0.25) (layer F.Cu) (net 11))
 (segment (start 133.926 83.508) (end 132.53 83.508) (width 0.25) (layer F.Cu) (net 11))
 (segment (start 132.53 83.508) (end 131.699 82.677) (width 0.25) (layer F.Cu) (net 11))
 (segment (start 131.699 82.677) (end 129.794 82.677) (width 0.25) (layer F.Cu) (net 11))
 (segment (start 129.794 82.677) (end 129.222 82.1055) (width 0.25) (layer F.Cu) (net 11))
 (segment (start 129.222 82.1055) (end 129.222 80.2005) (width 0.25) (layer F.Cu) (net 11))
 (segment (start 136.502 85.8045) (end 136.502 85.4485) (width 0.25) (layer F.Cu) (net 12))
 (segment (start 136.502 85.4485) (end 134.112 83.058) (width 0.25) (layer F.Cu) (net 12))
 (segment (start 134.112 83.058) (end 132.842 83.058) (width 0.25) (layer F.Cu) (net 12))
 (segment (start 132.842 83.058) (end 131.762 81.9785) (width 0.25) (layer F.Cu) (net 12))
 (segment (start 131.762 81.9785) (end 131.762 80.2005) (width 0.25) (layer F.Cu) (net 12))
 (segment (start 132.102 85.8045) (end 130.762 85.8045) (width 0.25) (layer F.Cu) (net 13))
 (segment (start 130.762 85.8045) (end 129.159 84.201) (width 0.25) (layer F.Cu) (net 13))
 (segment (start 129.159 84.201) (end 129.921 83.439) (width 0.25) (layer B.Cu) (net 13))
 (segment (start 129.921 83.439) (end 131.826 83.439) (width 0.25) (layer B.Cu) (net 13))
 (segment (start 131.826 83.439) (end 133.35 81.915) (width 0.25) (layer B.Cu) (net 13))
 (segment (start 133.35 81.915) (end 133.985 81.915) (width 0.25) (layer B.Cu) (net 13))
 (segment (start 133.985 81.915) (end 134.302 81.5975) (width 0.25) (layer B.Cu) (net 13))
 (segment (start 134.302 81.5975) (end 134.302 80.2005) (width 0.25) (layer B.Cu) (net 13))
 (via (at 129.159 84.201) (size 0.6) (layers F.Cu B.Cu) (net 13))
 (segment (start 132.102 86.3045) (end 130.246 86.3045) (width 0.25) (layer F.Cu) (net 14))
 (segment (start 130.246 86.3045) (end 129.286 85.344) (width 0.25) (layer F.Cu) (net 14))
 (segment (start 129.286 85.344) (end 130.683 83.947) (width 0.25) (layer B.Cu) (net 14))
 (segment (start 130.683 83.947) (end 134.62 83.947) (width 0.25) (layer B.Cu) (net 14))
 (segment (start 134.62 83.947) (end 136.842 81.7245) (width 0.25) (layer B.Cu) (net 14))
 (segment (start 136.842 81.7245) (end 136.842 80.2005) (width 0.25) (layer B.Cu) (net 14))
 (via (at 129.286 85.344) (size 0.6) (layers F.Cu B.Cu) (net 14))
 (segment (start 114.935 108.204) (end 120.904 108.204) (width 0.5) (layer F.Cu) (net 3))
 (segment (start 120.904 108.204) (end 124.46 104.648) (width 0.5) (layer F.Cu) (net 3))
 (segment (start 124.46 104.648) (end 124.46 100.076) (width 0.5) (layer F.Cu) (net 3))
 (segment (start 124.46 100.076) (end 126.238 98.298) (width 0.5) (layer F.Cu) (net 3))
 (segment (start 126.238 98.298) (end 127.889 98.298) (width 0.5) (layer F.Cu) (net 3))
 (segment (start 127.889 98.298) (end 129.921 98.298) (width 0.5) (layer F.Cu) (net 3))
 (segment (start 129.921 98.298) (end 131.064 99.441) (width 0.5) (layer F.Cu) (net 3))
 (segment (start 131.064 99.441) (end 131.064 101.854) (width 0.5) (layer F.Cu) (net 3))
 (segment (start 131.064 101.854) (end 132.048 102.838) (width 0.5) (layer F.Cu) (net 3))
 (segment (start 132.048 102.838) (end 133.096 102.838) (width 0.5) (layer F.Cu) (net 3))
 (segment (start 131.5721 109.197) (end 131.572 109.1971) (width 0.25) (layer F.Cu) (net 4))
 (segment (start 131.5721 109.197) (end 133.073 109.197) (width 0.5) (layer F.Cu) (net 4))
 (segment (start 133.073 109.197) (end 133.858 109.982) (width 0.5) (layer F.Cu) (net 4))
 (segment (start 133.858 109.982) (end 133.858 112.014) (width 0.5) (layer F.Cu) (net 4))
 (segment (start 133.858 112.014) (end 134.334 112.49) (width 0.5) (layer F.Cu) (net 4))
 (segment (start 134.334 112.49) (end 136.144 112.49) (width 0.5) (layer F.Cu) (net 4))
 (segment (start 131.572 109.197) (end 131.5721 109.197) (width 0.5) (layer F.Cu) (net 4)))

